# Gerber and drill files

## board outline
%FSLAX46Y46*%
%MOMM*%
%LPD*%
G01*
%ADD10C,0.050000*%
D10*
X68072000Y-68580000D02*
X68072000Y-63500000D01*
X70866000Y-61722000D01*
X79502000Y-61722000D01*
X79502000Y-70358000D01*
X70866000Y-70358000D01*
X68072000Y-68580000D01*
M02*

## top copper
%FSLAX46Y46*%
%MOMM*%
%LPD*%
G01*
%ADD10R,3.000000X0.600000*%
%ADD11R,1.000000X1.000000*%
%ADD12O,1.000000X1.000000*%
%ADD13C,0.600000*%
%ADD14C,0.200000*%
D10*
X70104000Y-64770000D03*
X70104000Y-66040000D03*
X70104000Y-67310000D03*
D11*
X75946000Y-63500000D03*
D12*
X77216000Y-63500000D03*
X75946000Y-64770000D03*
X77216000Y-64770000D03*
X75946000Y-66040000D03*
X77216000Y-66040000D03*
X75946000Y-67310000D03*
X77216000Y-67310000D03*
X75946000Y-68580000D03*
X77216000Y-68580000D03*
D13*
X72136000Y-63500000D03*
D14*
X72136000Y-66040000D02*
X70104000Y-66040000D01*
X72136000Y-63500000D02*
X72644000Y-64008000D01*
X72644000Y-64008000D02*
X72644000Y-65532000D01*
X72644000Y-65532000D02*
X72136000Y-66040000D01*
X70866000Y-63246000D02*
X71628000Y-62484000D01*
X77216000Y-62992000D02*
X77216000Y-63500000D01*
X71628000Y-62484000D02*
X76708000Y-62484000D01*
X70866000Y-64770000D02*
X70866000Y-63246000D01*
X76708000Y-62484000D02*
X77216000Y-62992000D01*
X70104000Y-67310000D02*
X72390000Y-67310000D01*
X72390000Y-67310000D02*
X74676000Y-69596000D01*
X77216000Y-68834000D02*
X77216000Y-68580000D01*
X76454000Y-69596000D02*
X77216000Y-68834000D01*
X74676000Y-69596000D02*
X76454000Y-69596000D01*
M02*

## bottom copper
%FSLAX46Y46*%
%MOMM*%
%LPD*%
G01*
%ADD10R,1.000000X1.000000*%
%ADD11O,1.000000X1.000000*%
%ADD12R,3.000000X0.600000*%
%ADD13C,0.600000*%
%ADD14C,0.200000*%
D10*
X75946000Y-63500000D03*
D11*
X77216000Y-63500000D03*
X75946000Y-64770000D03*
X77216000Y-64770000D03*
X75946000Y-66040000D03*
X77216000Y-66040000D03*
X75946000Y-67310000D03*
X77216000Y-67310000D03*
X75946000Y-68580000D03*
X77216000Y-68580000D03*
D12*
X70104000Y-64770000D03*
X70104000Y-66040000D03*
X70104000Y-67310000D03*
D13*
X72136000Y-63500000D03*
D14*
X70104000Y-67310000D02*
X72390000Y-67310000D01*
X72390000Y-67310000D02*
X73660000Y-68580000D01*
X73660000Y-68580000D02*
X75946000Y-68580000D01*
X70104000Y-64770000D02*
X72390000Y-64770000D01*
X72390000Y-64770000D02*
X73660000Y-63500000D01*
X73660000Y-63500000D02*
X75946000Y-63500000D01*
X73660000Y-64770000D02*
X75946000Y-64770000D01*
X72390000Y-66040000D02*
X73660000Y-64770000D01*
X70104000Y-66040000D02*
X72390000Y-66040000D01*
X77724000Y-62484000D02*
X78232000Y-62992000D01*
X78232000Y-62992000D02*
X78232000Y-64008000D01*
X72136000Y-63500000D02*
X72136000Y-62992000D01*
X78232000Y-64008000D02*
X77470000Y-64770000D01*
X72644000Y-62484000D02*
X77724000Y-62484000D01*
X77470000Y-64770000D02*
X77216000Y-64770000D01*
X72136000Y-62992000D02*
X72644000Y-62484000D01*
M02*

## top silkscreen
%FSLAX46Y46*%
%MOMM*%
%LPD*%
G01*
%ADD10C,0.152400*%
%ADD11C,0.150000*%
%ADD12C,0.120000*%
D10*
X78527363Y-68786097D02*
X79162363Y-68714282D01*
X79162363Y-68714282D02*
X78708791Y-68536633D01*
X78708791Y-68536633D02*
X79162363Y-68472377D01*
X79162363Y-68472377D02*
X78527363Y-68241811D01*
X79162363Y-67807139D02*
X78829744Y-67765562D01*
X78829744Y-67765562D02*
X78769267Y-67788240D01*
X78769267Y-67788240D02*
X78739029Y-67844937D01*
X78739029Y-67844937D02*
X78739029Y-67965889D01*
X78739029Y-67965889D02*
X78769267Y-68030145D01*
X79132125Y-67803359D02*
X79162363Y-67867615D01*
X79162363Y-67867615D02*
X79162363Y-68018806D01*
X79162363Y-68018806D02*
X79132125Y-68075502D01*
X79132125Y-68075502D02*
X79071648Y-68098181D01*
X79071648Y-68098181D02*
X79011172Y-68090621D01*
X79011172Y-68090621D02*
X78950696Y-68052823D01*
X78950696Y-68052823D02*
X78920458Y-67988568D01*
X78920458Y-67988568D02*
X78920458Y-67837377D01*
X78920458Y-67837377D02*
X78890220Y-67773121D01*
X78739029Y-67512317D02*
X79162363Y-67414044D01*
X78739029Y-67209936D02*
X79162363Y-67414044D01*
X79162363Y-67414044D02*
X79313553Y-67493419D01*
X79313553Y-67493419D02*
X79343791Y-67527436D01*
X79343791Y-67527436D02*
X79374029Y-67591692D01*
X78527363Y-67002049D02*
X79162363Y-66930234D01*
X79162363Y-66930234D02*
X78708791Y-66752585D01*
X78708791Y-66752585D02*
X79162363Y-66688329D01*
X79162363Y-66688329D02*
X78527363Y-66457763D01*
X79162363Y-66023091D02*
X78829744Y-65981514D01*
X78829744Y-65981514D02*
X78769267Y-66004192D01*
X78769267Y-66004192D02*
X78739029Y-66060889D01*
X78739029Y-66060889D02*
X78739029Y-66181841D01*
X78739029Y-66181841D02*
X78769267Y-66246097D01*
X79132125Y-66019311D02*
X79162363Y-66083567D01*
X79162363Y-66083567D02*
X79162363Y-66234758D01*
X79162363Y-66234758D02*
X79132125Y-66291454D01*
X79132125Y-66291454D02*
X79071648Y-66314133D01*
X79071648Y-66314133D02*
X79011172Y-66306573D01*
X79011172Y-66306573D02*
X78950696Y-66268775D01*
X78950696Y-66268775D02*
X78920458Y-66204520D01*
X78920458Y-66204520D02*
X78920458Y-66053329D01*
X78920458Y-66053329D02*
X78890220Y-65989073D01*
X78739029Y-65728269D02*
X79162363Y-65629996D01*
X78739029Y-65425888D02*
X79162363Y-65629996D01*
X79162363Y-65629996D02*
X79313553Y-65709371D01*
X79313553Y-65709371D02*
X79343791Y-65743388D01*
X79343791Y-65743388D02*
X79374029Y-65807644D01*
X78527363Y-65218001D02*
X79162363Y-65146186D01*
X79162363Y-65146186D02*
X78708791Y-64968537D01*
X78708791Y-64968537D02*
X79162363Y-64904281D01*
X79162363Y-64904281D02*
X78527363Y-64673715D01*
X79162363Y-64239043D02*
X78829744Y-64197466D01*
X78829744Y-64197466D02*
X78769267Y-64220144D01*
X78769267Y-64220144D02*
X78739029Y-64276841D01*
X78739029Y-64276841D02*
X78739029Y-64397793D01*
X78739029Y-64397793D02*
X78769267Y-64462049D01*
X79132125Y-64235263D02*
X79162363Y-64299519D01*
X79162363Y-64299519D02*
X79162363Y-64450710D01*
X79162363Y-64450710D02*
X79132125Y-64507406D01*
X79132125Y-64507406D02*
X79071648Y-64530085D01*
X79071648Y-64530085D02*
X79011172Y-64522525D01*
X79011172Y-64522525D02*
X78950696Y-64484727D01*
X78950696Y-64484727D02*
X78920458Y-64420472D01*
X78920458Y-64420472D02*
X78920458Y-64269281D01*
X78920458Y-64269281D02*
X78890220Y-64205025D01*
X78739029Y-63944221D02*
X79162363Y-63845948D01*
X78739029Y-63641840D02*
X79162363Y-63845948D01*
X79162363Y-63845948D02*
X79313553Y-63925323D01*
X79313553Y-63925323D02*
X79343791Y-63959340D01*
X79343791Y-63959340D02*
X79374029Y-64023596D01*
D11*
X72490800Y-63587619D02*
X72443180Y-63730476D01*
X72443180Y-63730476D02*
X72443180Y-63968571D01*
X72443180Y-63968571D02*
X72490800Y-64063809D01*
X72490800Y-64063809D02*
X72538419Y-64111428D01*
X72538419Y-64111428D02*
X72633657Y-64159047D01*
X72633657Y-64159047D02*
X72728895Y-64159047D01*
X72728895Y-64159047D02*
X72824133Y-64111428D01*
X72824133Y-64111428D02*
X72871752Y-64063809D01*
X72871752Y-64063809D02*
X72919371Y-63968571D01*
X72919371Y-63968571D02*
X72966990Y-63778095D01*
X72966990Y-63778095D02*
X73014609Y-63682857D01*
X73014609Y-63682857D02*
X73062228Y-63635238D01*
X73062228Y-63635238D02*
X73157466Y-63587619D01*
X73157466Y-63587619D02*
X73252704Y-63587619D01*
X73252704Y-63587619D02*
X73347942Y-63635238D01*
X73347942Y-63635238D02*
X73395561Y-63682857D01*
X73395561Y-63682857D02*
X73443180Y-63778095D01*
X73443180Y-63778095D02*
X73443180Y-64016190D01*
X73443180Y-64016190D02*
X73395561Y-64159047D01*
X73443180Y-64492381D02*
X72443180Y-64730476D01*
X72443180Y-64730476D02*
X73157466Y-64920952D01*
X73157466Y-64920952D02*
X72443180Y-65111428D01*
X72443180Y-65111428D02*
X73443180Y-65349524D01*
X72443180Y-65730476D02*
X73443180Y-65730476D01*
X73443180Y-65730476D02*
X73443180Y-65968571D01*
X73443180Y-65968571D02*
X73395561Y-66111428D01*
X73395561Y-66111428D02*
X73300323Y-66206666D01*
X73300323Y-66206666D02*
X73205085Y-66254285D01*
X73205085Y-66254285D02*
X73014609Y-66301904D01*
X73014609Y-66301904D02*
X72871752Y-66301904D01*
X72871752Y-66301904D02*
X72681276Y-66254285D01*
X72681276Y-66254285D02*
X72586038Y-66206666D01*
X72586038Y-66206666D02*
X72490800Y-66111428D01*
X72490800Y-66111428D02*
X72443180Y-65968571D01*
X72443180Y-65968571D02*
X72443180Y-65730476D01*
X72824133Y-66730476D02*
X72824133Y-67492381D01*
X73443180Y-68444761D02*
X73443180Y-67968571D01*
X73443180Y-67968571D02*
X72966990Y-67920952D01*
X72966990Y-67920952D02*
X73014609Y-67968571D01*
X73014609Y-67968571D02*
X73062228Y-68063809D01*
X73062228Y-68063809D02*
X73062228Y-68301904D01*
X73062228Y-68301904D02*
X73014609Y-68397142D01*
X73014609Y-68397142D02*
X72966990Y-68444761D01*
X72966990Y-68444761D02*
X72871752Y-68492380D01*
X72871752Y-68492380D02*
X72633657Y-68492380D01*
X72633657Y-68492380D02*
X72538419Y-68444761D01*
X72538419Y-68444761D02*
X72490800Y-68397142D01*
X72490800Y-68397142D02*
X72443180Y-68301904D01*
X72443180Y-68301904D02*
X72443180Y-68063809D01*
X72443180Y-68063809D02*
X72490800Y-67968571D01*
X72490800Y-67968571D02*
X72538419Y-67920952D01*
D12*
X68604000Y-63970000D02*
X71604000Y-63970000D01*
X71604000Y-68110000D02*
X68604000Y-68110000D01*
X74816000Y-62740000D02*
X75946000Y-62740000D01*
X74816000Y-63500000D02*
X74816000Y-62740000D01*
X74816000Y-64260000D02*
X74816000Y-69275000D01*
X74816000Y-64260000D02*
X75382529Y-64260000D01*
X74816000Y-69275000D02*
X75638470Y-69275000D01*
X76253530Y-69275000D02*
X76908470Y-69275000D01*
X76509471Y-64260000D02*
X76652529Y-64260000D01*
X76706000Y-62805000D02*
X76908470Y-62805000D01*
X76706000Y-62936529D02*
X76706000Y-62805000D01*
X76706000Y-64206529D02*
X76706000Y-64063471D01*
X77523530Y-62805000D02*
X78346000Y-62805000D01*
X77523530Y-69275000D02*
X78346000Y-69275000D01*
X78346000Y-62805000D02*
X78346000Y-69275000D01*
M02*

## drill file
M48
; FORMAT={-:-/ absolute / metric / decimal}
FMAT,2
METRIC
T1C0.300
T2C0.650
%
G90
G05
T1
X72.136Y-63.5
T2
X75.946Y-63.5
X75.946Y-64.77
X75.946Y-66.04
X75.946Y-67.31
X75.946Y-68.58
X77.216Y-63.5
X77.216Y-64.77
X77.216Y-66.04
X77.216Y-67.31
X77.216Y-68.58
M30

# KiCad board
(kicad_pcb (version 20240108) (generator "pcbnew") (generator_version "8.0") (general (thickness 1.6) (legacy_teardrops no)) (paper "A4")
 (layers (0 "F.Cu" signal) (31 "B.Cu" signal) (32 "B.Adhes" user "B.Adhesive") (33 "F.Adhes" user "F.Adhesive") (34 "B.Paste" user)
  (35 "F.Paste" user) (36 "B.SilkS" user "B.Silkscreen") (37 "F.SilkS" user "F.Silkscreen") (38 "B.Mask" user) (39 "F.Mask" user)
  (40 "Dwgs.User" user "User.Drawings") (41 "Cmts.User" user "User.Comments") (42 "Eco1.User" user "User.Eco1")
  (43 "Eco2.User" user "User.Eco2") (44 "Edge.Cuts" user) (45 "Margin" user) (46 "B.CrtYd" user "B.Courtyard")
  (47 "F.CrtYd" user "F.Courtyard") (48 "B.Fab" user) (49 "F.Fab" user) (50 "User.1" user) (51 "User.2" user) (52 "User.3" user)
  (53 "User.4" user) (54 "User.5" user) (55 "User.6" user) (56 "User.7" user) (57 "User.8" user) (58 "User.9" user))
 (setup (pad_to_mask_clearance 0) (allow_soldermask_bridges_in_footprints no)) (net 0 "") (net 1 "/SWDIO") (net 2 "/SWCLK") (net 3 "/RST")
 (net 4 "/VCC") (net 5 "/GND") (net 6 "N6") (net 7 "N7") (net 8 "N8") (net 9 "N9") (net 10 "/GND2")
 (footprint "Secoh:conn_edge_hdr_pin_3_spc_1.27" (layer "F.Cu") (at 70.104 66.04 -90)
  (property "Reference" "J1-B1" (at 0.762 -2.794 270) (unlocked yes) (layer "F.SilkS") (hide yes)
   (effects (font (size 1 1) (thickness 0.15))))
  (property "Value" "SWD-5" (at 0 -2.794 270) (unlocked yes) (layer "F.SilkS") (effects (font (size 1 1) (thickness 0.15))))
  (fp_line (start -2.07 1.5) (end -2.07 -1.5) (stroke (width 0.12) (type default)) (layer "F.SilkS"))
  (fp_line (start 2.07 -1.5) (end 2.07 1.5) (stroke (width 0.12) (type default)) (layer "F.SilkS"))
  (pad "1" smd rect (at -1.27 0 270) (size 0.6 3) (layers "F.Cu" "F.Paste" "F.Mask") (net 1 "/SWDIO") (thermal_bridge_angle 45))
  (pad "2" smd rect (at 0 0 270) (size 0.6 3) (layers "F.Cu" "F.Paste" "F.Mask") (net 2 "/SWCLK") (thermal_bridge_angle 45))
  (pad "3" smd rect (at 1.27 0 270) (size 0.6 3) (layers "F.Cu" "F.Paste" "F.Mask") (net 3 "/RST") (thermal_bridge_angle 45)))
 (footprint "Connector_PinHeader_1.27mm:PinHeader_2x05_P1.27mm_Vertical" (layer "F.Cu") (at 75.946 63.5)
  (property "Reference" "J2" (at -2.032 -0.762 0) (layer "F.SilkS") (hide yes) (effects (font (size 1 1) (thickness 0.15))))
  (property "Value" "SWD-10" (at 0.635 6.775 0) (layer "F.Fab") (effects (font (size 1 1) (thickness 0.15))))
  (fp_line (start -1.13 -0.76) (end 0 -0.76) (stroke (width 0.12) (type solid)) (layer "F.SilkS"))
  (fp_line (start -1.13 0) (end -1.13 -0.76) (stroke (width 0.12) (type solid)) (layer "F.SilkS"))
  (fp_line (start -1.13 0.76) (end -1.13 5.775) (stroke (width 0.12) (type solid)) (layer "F.SilkS"))
  (fp_line (start -1.13 0.76) (end -0.563471 0.76) (stroke (width 0.12) (type solid)) (layer "F.SilkS"))
  (fp_line (start -1.13 5.775) (end -0.30753 5.775) (stroke (width 0.12) (type solid)) (layer "F.SilkS"))
  (fp_line (start 0.30753 5.775) (end 0.96247 5.775) (stroke (width 0.12) (type solid)) (layer "F.SilkS"))
  (fp_line (start 0.563471 0.76) (end 0.706529 0.76) (stroke (width 0.12) (type solid)) (layer "F.SilkS"))
  (fp_line (start 0.76 -0.695) (end 0.96247 -0.695) (stroke (width 0.12) (type solid)) (layer "F.SilkS"))
  (fp_line (start 0.76 -0.563471) (end 0.76 -0.695) (stroke (width 0.12) (type solid)) (layer "F.SilkS"))
  (fp_line (start 0.76 0.706529) (end 0.76 0.563471) (stroke (width 0.12) (type solid)) (layer "F.SilkS"))
  (fp_line (start 1.57753 -0.695) (end 2.4 -0.695) (stroke (width 0.12) (type solid)) (layer "F.SilkS"))
  (fp_line (start 1.57753 5.775) (end 2.4 5.775) (stroke (width 0.12) (type solid)) (layer "F.SilkS"))
  (fp_line (start 2.4 -0.695) (end 2.4 5.775) (stroke (width 0.12) (type solid)) (layer "F.SilkS"))
  (pad "1" thru_hole rect (at 0 0) (size 1 1) (drill 0.65) (layers "*.Cu" "*.Mask") (remove_unused_layers no) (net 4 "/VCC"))
  (pad "2" thru_hole oval (at 1.27 0) (size 1 1) (drill 0.65) (layers "*.Cu" "*.Mask") (remove_unused_layers no) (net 1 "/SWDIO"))
  (pad "3" thru_hole oval (at 0 1.27) (size 1 1) (drill 0.65) (layers "*.Cu" "*.Mask") (remove_unused_layers no) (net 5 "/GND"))
  (pad "4" thru_hole oval (at 1.27 1.27) (size 1 1) (drill 0.65) (layers "*.Cu" "*.Mask") (remove_unused_layers no) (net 2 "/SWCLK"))
  (pad "5" thru_hole oval (at 0 2.54) (size 1 1) (drill 0.65) (layers "*.Cu" "*.Mask") (remove_unused_layers no) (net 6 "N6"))
  (pad "6" thru_hole oval (at 1.27 2.54) (size 1 1) (drill 0.65) (layers "*.Cu" "*.Mask") (remove_unused_layers no) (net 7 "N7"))
  (pad "7" thru_hole oval (at 0 3.81) (size 1 1) (drill 0.65) (layers "*.Cu" "*.Mask") (remove_unused_layers no) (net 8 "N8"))
  (pad "8" thru_hole oval (at 1.27 3.81) (size 1 1) (drill 0.65) (layers "*.Cu" "*.Mask") (remove_unused_layers no) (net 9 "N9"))
  (pad "9" thru_hole oval (at 0 5.08) (size 1 1) (drill 0.65) (layers "*.Cu" "*.Mask") (remove_unused_layers no) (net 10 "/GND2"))
  (pad "10" thru_hole oval (at 1.27 5.08) (size 1 1) (drill 0.65) (layers "*.Cu" "*.Mask") (remove_unused_layers no) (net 3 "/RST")))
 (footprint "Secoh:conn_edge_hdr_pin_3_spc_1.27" (layer "B.Cu") (at 70.104 66.04 -90)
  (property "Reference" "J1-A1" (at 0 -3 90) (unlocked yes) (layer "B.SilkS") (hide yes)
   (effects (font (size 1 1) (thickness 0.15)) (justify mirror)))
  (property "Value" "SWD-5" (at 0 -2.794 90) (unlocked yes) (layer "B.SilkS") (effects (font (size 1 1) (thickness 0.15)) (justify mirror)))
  (pad "1" smd rect (at -1.27 0 270) (size 0.6 3) (layers "B.Cu" "B.Paste" "B.Mask") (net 4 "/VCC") (thermal_bridge_angle 45))
  (pad "2" smd rect (at 0 0 270) (size 0.6 3) (layers "B.Cu" "B.Paste" "B.Mask") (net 5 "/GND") (thermal_bridge_angle 45))
  (pad "3" smd rect (at 1.27 0 270) (size 0.6 3) (layers "B.Cu" "B.Paste" "B.Mask") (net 10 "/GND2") (thermal_bridge_angle 45)))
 (gr_poly
  (pts (xy 68.072 68.58) (xy 68.072 63.5) (xy 70.866 61.722) (xy 79.502 61.722) (xy 79.502 70.358) (xy 70.866 70.358))
  (stroke (width 0.05) (type solid)) (fill none) (layer "Edge.Cuts"))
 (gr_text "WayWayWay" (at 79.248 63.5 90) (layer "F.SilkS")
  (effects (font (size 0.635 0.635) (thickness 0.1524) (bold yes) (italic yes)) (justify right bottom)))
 (segment (start 70.104 67.31) (end 72.39 67.31) (width 0.2) (layer "B.Cu") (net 10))
 (segment (start 72.39 67.31) (end 73.66 68.58) (width 0.2) (layer "B.Cu") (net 10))
 (segment (start 73.66 68.58) (end 75.946 68.58) (width 0.2) (layer "B.Cu") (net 10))
 (segment (start 70.104 64.77) (end 72.39 64.77) (width 0.2) (layer "B.Cu") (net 4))
 (segment (start 72.39 64.77) (end 73.66 63.5) (width 0.2) (layer "B.Cu") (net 4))
 (segment (start 73.66 63.5) (end 75.946 63.5) (width 0.2) (layer "B.Cu") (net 4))
 (segment (start 73.66 64.77) (end 75.946 64.77) (width 0.2) (layer "B.Cu") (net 5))
 (segment (start 72.39 66.04) (end 73.66 64.77) (width 0.2) (layer "B.Cu") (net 5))
 (segment (start 70.104 66.04) (end 72.39 66.04) (width 0.2) (layer "B.Cu") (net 5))
 (segment (start 72.136 66.04) (end 70.104 66.04) (width 0.2) (layer "F.Cu") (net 2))
 (segment (start 72.136 63.5) (end 72.644 64.008) (width 0.2) (layer "F.Cu") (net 2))
 (segment (start 72.644 64.008) (end 72.644 65.532) (width 0.2) (layer "F.Cu") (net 2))
 (segment (start 72.644 65.532) (end 72.136 66.04) (width 0.2) (layer "F.Cu") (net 2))
 (via (at 72.136 63.5) (size 0.6) (drill 0.3) (layers "F.Cu" "B.Cu") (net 2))
 (segment (start 77.724 62.484) (end 78.232 62.992) (width 0.2) (layer "B.Cu") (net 2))
 (segment (start 78.232 62.992) (end 78.232 64.008) (width 0.2) (layer "B.Cu") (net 2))
 (segment (start 72.136 63.5) (end 72.136 62.992) (width 0.2) (layer "B.Cu") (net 2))
 (segment (start 78.232 64.008) (end 77.47 64.77) (width 0.2) (layer "B.Cu") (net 2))
 (segment (start 72.644 62.484) (end 77.724 62.484) (width 0.2) (layer "B.Cu") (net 2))
 (segment (start 77.47 64.77) (end 77.216 64.77) (width 0.2) (layer "B.Cu") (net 2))
 (segment (start 72.136 62.992) (end 72.644 62.484) (width 0.2) (layer "B.Cu") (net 2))
 (segment (start 70.866 63.246) (end 71.628 62.484) (width 0.2) (layer "F.Cu") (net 1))
 (segment (start 77.216 62.992) (end 77.216 63.5) (width 0.2) (layer "F.Cu") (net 1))
 (segment (start 71.628 62.484) (end 76.708 62.484) (width 0.2) (layer "F.Cu") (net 1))
 (segment (start 70.866 64.77) (end 70.866 63.246) (width 0.2) (layer "F.Cu") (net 1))
 (segment (start 76.708 62.484) (end 77.216 62.992) (width 0.2) (layer "F.Cu") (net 1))
 (segment (start 70.104 67.31) (end 72.39 67.31) (width 0.2) (layer "F.Cu") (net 3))
 (segment (start 72.39 67.31) (end 74.676 69.596) (width 0.2) (layer "F.Cu") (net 3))
 (segment (start 77.216 68.834) (end 77.216 68.58) (width 0.2) (layer "F.Cu") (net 3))
 (segment (start 76.454 69.596) (end 77.216 68.834) (width 0.2) (layer "F.Cu") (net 3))
 (segment (start 74.676 69.596) (end 76.454 69.596) (width 0.2) (layer "F.Cu") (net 3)))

